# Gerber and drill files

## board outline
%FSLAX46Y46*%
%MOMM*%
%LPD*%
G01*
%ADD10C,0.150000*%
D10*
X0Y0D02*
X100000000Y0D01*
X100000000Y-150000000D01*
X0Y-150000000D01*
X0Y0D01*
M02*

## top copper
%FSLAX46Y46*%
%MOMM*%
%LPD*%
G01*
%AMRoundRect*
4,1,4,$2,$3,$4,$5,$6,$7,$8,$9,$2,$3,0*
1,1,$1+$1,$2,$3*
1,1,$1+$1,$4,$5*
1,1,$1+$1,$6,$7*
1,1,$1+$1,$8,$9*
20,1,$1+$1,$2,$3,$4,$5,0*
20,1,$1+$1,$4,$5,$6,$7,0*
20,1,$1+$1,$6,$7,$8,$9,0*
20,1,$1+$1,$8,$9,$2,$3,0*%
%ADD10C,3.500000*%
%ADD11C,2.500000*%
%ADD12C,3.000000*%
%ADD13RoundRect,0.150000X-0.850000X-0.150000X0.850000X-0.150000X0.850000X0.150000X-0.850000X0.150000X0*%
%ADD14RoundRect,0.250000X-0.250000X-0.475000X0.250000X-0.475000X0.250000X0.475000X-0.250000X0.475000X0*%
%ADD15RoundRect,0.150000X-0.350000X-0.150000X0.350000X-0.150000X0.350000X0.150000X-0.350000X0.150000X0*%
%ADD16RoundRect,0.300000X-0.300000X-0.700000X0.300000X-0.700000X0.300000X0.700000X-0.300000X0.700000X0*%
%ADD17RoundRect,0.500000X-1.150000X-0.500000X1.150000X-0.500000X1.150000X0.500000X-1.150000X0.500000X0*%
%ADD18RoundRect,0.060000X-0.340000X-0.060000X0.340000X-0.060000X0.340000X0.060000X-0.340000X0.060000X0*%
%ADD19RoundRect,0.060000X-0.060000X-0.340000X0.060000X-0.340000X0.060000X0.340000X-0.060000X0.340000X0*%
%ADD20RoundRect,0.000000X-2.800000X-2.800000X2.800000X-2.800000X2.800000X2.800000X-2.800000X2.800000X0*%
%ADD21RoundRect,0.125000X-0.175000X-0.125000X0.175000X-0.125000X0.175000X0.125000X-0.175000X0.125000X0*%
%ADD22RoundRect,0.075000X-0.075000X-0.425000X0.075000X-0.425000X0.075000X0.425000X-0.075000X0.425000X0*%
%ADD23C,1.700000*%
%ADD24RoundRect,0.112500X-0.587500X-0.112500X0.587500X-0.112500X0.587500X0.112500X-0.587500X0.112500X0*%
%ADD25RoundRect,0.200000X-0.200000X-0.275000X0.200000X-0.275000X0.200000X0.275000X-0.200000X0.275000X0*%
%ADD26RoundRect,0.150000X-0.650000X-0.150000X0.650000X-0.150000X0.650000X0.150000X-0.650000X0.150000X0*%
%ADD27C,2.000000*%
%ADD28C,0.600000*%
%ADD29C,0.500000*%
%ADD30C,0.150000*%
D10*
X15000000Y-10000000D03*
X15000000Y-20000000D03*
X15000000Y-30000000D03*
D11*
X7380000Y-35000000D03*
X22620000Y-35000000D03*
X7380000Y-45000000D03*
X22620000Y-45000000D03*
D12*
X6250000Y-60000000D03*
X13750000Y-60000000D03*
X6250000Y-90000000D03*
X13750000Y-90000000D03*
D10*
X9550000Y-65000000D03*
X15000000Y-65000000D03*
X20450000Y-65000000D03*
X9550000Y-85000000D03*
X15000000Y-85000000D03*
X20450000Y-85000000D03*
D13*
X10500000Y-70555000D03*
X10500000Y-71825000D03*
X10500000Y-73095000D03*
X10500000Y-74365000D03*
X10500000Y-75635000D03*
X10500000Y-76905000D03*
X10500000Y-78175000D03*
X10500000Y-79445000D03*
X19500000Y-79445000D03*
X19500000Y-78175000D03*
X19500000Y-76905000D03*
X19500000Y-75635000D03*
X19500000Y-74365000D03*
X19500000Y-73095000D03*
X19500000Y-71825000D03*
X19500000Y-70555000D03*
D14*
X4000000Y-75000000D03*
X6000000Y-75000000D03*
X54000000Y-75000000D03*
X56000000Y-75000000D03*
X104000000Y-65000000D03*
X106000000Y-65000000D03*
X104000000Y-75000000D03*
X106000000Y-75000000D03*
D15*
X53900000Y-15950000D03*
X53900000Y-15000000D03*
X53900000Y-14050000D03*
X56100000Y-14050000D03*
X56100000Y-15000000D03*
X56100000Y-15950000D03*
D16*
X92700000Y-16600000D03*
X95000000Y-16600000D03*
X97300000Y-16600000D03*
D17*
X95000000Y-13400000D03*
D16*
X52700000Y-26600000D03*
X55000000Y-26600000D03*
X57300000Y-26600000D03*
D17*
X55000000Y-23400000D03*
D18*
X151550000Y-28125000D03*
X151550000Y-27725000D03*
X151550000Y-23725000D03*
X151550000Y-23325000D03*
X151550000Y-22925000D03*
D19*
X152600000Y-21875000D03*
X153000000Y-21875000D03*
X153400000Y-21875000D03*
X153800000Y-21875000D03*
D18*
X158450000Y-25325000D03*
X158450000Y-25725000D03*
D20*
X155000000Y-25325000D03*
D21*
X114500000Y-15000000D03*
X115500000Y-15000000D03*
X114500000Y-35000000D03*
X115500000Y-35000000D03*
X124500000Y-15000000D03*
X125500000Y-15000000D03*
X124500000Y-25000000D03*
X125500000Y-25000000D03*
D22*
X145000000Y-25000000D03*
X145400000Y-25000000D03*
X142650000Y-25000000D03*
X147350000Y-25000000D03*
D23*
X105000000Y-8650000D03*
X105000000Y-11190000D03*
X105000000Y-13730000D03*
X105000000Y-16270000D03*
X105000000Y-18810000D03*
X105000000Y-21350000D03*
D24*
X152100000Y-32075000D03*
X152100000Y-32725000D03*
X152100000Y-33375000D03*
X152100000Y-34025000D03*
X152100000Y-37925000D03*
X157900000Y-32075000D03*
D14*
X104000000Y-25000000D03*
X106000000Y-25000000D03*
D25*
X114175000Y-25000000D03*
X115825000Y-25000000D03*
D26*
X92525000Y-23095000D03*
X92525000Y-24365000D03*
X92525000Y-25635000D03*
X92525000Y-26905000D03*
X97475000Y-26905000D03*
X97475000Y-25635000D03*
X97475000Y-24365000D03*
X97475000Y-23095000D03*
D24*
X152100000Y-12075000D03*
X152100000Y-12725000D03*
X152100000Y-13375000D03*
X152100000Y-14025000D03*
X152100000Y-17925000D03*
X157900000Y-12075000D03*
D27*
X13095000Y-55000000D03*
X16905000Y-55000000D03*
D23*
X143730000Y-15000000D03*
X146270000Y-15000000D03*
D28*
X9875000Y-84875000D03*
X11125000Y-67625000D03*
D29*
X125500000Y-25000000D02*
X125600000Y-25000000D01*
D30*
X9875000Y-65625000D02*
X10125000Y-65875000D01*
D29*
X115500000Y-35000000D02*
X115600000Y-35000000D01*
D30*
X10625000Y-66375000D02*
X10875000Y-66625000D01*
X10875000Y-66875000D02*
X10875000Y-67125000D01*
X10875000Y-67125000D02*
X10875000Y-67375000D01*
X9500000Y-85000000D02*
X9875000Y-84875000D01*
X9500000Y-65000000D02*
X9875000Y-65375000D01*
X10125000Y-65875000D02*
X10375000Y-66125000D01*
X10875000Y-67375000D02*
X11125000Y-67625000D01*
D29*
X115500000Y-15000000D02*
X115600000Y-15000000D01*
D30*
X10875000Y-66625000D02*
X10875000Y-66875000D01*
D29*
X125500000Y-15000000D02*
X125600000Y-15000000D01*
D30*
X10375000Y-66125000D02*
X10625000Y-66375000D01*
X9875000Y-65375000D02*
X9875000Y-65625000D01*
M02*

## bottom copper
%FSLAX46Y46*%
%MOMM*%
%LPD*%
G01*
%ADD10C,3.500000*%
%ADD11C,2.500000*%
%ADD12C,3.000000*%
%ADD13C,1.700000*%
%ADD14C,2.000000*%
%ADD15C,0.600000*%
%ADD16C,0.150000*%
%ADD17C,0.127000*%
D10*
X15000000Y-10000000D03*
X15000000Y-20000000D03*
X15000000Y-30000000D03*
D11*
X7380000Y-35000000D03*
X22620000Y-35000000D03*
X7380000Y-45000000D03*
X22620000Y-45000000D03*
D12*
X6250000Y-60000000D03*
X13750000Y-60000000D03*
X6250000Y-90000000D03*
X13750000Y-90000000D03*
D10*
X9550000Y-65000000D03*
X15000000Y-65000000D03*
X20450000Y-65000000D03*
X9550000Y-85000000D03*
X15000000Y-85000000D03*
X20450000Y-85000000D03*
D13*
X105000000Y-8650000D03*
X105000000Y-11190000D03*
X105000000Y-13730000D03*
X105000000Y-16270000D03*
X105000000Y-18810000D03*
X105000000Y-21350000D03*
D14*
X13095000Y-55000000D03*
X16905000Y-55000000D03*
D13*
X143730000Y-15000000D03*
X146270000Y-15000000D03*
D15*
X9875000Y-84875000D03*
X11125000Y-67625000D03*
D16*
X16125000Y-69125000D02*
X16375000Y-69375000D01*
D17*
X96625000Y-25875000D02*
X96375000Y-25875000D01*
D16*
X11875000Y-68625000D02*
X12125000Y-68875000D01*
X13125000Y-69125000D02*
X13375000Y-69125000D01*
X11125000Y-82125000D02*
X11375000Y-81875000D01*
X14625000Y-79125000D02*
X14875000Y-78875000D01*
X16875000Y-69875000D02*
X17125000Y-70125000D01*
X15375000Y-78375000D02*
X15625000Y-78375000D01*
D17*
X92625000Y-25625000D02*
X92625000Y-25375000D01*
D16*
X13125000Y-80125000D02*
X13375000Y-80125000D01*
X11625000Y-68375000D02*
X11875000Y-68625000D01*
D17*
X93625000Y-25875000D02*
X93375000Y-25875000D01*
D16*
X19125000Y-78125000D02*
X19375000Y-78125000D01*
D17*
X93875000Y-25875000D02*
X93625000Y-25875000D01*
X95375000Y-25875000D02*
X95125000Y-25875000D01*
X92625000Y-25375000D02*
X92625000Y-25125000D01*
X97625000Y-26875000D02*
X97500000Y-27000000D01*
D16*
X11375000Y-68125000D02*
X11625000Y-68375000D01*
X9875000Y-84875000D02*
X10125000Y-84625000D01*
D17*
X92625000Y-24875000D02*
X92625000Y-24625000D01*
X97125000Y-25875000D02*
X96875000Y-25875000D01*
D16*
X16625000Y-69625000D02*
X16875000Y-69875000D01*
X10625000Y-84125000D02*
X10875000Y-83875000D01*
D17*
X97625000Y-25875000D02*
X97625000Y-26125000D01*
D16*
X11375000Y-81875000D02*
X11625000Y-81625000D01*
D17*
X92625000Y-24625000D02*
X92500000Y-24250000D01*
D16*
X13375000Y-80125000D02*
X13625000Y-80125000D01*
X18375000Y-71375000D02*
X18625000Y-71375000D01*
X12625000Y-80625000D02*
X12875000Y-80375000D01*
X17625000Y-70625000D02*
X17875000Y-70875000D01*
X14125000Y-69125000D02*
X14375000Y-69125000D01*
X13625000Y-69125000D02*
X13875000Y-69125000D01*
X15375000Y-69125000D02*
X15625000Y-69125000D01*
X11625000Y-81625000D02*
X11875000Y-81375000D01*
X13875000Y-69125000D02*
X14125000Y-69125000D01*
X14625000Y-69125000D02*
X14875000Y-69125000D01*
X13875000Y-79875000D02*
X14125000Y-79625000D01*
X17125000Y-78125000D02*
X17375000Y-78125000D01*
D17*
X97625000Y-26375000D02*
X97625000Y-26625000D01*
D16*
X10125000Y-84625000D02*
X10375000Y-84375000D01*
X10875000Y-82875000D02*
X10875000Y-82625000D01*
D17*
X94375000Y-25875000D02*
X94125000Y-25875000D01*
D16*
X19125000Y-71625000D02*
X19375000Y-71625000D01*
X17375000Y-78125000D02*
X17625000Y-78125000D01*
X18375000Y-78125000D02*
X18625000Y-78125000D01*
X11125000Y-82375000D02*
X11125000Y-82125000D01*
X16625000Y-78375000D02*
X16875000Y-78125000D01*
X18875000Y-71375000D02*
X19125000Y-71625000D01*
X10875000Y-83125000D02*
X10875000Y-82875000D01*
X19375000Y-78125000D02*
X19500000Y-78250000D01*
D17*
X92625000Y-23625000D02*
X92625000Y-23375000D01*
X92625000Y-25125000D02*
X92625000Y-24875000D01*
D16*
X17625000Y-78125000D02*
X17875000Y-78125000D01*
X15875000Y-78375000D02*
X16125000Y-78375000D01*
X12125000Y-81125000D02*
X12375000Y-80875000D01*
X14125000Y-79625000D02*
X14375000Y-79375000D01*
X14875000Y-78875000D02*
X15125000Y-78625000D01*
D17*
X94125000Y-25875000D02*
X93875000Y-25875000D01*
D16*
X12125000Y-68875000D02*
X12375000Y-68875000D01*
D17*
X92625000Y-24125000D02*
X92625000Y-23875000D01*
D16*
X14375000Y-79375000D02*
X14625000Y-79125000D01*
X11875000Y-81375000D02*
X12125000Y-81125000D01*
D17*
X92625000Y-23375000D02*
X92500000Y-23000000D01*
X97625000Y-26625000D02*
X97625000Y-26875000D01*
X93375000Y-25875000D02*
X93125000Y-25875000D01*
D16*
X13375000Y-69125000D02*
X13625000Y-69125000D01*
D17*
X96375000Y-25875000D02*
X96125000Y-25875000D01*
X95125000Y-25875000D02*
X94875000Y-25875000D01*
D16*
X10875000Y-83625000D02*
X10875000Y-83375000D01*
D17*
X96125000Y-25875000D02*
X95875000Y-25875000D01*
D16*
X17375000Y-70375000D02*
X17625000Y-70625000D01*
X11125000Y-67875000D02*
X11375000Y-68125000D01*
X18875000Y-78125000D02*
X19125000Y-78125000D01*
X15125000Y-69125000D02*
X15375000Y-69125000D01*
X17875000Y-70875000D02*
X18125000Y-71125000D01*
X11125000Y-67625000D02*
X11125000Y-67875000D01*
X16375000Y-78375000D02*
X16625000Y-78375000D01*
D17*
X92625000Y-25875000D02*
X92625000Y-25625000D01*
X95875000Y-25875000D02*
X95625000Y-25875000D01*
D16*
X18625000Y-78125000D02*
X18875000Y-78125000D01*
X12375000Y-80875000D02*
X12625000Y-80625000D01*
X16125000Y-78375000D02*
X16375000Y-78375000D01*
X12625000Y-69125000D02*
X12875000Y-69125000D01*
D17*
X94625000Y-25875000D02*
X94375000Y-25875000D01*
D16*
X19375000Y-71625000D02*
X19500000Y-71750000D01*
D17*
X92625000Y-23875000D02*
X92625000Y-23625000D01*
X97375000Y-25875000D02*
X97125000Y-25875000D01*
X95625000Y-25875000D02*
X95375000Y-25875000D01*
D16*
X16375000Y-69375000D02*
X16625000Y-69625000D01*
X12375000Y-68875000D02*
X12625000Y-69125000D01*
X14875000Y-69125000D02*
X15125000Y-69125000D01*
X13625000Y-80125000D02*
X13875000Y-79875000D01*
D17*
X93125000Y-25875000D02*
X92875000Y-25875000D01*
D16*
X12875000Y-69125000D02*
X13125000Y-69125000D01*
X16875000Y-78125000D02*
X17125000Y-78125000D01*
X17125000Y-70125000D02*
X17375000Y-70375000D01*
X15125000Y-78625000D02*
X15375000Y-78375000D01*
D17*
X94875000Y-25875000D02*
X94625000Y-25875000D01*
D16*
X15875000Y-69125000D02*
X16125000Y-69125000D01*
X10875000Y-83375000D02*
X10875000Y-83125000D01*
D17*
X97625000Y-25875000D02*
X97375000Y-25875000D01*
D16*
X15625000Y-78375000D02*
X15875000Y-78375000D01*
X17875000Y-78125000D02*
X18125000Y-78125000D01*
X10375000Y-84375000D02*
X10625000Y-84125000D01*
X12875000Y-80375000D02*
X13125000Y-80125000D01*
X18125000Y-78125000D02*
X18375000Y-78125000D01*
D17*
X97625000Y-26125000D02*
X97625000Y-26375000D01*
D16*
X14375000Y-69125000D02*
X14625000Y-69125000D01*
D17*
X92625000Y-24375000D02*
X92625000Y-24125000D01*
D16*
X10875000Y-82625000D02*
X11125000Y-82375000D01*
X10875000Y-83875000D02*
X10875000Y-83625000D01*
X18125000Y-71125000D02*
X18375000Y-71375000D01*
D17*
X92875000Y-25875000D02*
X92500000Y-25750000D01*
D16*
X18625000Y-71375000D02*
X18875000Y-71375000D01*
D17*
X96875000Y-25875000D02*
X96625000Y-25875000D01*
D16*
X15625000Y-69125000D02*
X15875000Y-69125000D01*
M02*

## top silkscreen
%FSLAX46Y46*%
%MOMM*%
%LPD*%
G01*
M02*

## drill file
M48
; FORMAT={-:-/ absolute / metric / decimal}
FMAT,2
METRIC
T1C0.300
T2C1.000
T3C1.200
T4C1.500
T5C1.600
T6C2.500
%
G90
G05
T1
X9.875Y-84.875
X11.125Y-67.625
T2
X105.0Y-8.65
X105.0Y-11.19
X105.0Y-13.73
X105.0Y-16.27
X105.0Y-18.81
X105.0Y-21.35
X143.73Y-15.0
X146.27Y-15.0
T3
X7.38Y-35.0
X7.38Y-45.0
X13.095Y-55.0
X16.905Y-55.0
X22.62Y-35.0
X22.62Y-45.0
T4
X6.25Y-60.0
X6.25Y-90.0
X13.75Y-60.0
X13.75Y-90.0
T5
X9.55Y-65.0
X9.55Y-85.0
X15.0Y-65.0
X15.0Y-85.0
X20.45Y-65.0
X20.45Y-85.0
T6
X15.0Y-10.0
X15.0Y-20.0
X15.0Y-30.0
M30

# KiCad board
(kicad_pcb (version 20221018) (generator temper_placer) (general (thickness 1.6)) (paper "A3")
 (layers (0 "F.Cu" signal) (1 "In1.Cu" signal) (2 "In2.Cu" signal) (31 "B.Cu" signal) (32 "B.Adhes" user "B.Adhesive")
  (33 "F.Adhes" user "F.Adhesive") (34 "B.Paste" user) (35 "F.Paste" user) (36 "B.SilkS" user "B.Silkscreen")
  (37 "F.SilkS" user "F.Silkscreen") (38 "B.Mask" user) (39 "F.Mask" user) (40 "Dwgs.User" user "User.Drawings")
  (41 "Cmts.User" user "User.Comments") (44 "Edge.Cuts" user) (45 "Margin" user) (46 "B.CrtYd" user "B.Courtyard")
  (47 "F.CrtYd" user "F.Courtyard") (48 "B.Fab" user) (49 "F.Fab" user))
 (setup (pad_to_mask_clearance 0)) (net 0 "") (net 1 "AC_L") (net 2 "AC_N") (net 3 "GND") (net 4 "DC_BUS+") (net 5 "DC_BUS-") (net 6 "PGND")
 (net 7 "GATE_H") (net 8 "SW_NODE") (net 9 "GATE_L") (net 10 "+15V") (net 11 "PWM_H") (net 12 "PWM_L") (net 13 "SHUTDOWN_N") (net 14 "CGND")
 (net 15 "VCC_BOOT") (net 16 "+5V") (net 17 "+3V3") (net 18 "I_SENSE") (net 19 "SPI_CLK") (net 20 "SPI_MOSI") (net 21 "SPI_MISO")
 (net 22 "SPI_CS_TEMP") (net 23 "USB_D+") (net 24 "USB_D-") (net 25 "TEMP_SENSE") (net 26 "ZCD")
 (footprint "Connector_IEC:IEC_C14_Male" (layer "F.Cu") (at 15 10 0) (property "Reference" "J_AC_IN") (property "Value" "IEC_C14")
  (pad "1" thru_hole circle (at 0 0) (size 3.5 3.5) (drill 2.5) (layers *.Cu *.Mask) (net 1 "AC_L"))
  (pad "2" thru_hole circle (at 0 10) (size 3.5 3.5) (drill 2.5) (layers *.Cu *.Mask) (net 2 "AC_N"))
  (pad "3" thru_hole circle (at 0 20) (size 3.5 3.5) (drill 2.5) (layers *.Cu *.Mask) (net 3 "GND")))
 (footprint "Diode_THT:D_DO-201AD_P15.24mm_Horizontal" (layer "F.Cu") (at 7.38 35 0) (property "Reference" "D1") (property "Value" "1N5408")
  (pad "1" thru_hole circle (at 0 0) (size 2.5 2.5) (drill 1.2) (layers *.Cu *.Mask) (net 1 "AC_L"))
  (pad "2" thru_hole circle (at 15.24 0) (size 2.5 2.5) (drill 1.2) (layers *.Cu *.Mask) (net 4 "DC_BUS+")))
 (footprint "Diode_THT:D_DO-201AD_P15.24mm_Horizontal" (layer "F.Cu") (at 7.38 45 0) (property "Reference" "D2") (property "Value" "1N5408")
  (pad "1" thru_hole circle (at 0 0) (size 2.5 2.5) (drill 1.2) (layers *.Cu *.Mask) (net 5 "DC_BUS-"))
  (pad "2" thru_hole circle (at 15.24 0) (size 2.5 2.5) (drill 1.2) (layers *.Cu *.Mask) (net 2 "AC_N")))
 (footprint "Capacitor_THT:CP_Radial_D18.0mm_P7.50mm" (layer "F.Cu") (at 6.25 60 0) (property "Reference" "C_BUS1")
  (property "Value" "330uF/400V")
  (pad "1" thru_hole circle (at 0 0) (size 3 3) (drill 1.5) (layers *.Cu *.Mask) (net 4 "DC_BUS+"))
  (pad "2" thru_hole circle (at 7.5 0) (size 3 3) (drill 1.5) (layers *.Cu *.Mask) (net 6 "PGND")))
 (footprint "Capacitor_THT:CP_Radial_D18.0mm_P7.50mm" (layer "F.Cu") (at 6.25 90 0) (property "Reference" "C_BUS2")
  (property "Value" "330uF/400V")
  (pad "1" thru_hole circle (at 0 0) (size 3 3) (drill 1.5) (layers *.Cu *.Mask) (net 6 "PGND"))
  (pad "2" thru_hole circle (at 7.5 0) (size 3 3) (drill 1.5) (layers *.Cu *.Mask) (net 5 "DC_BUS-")))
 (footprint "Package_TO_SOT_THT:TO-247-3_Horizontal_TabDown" (layer "F.Cu") (at 9.55 65 0) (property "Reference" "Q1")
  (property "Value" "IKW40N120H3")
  (pad "1" thru_hole circle (at 0 0) (size 3.5 3.5) (drill 1.6) (layers *.Cu *.Mask) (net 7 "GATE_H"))
  (pad "2" thru_hole circle (at 5.45 0) (size 3.5 3.5) (drill 1.6) (layers *.Cu *.Mask) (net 4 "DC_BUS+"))
  (pad "3" thru_hole circle (at 10.9 0) (size 3.5 3.5) (drill 1.6) (layers *.Cu *.Mask) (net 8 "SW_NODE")))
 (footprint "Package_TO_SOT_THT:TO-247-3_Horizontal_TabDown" (layer "F.Cu") (at 9.55 85 0) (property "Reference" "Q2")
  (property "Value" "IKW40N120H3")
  (pad "1" thru_hole circle (at 0 0) (size 3.5 3.5) (drill 1.6) (layers *.Cu *.Mask) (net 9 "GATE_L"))
  (pad "2" thru_hole circle (at 5.45 0) (size 3.5 3.5) (drill 1.6) (layers *.Cu *.Mask) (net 8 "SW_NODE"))
  (pad "3" thru_hole circle (at 10.9 0) (size 3.5 3.5) (drill 1.6) (layers *.Cu *.Mask) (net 5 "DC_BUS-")))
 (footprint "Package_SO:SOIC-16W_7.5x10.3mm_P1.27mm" (layer "F.Cu") (at 15 75 0) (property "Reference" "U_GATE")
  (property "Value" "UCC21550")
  (pad "1" smd roundrect (at -4.5 -4.445) (size 2 0.6) (layers "F.Cu" "F.Paste" "F.Mask") (roundrect_rratio 0.25) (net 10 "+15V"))
  (pad "2" smd roundrect (at -4.5 -3.175) (size 2 0.6) (layers "F.Cu" "F.Paste" "F.Mask") (roundrect_rratio 0.25) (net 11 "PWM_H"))
  (pad "3" smd roundrect (at -4.5 -1.905) (size 2 0.6) (layers "F.Cu" "F.Paste" "F.Mask") (roundrect_rratio 0.25) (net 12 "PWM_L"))
  (pad "4" smd roundrect (at -4.5 -0.635) (size 2 0.6) (layers "F.Cu" "F.Paste" "F.Mask") (roundrect_rratio 0.25) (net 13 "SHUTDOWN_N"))
  (pad "5" smd roundrect (at -4.5 0.635) (size 2 0.6) (layers "F.Cu" "F.Paste" "F.Mask") (roundrect_rratio 0.25) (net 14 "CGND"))
  (pad "6" smd roundrect (at -4.5 1.905) (size 2 0.6) (layers "F.Cu" "F.Paste" "F.Mask") (roundrect_rratio 0.25) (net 14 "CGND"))
  (pad "7" smd roundrect (at -4.5 3.175) (size 2 0.6) (layers "F.Cu" "F.Paste" "F.Mask") (roundrect_rratio 0.25) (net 14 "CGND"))
  (pad "8" smd roundrect (at -4.5 4.445) (size 2 0.6) (layers "F.Cu" "F.Paste" "F.Mask") (roundrect_rratio 0.25) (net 14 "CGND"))
  (pad "9" smd roundrect (at 4.5 4.445) (size 2 0.6) (layers "F.Cu" "F.Paste" "F.Mask") (roundrect_rratio 0.25) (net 8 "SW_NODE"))
  (pad "10" smd roundrect (at 4.5 3.175) (size 2 0.6) (layers "F.Cu" "F.Paste" "F.Mask") (roundrect_rratio 0.25) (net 9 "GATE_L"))
  (pad "11" smd roundrect (at 4.5 1.905) (size 2 0.6) (layers "F.Cu" "F.Paste" "F.Mask") (roundrect_rratio 0.25) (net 10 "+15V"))
  (pad "12" smd roundrect (at 4.5 0.635) (size 2 0.6) (layers "F.Cu" "F.Paste" "F.Mask") (roundrect_rratio 0.25) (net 6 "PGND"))
  (pad "13" smd roundrect (at 4.5 -0.635) (size 2 0.6) (layers "F.Cu" "F.Paste" "F.Mask") (roundrect_rratio 0.25) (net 6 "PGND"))
  (pad "14" smd roundrect (at 4.5 -1.905) (size 2 0.6) (layers "F.Cu" "F.Paste" "F.Mask") (roundrect_rratio 0.25) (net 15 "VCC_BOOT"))
  (pad "15" smd roundrect (at 4.5 -3.175) (size 2 0.6) (layers "F.Cu" "F.Paste" "F.Mask") (roundrect_rratio 0.25) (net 7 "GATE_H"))
  (pad "16" smd roundrect (at 4.5 -4.445) (size 2 0.6) (layers "F.Cu" "F.Paste" "F.Mask") (roundrect_rratio 0.25) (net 8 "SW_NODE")))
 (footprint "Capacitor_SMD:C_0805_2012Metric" (layer "F.Cu") (at 5 75 0) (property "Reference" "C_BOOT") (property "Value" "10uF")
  (pad "1" smd roundrect (at -1 0) (size 1 1.45) (layers "F.Cu" "F.Paste" "F.Mask") (roundrect_rratio 0.25) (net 15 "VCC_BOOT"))
  (pad "2" smd roundrect (at 1 0) (size 1 1.45) (layers "F.Cu" "F.Paste" "F.Mask") (roundrect_rratio 0.25) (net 8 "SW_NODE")))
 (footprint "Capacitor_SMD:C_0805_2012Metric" (layer "F.Cu") (at 55 75 0) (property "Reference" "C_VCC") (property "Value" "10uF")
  (pad "1" smd roundrect (at -1 0) (size 1 1.45) (layers "F.Cu" "F.Paste" "F.Mask") (roundrect_rratio 0.25) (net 10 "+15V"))
  (pad "2" smd roundrect (at 1 0) (size 1 1.45) (layers "F.Cu" "F.Paste" "F.Mask") (roundrect_rratio 0.25) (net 14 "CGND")))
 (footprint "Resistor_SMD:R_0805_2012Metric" (layer "F.Cu") (at 105 65 0) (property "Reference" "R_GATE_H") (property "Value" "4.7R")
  (pad "1" smd roundrect (at -1 0) (size 1 1.45) (layers "F.Cu" "F.Paste" "F.Mask") (roundrect_rratio 0.25) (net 7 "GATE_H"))
  (pad "2" smd roundrect (at 1 0) (size 1 1.45) (layers "F.Cu" "F.Paste" "F.Mask") (roundrect_rratio 0.25) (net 7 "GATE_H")))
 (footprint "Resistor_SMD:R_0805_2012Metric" (layer "F.Cu") (at 105 75 0) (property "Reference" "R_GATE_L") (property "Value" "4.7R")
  (pad "1" smd roundrect (at -1 0) (size 1 1.45) (layers "F.Cu" "F.Paste" "F.Mask") (roundrect_rratio 0.25) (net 9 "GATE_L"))
  (pad "2" smd roundrect (at 1 0) (size 1 1.45) (layers "F.Cu" "F.Paste" "F.Mask") (roundrect_rratio 0.25) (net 9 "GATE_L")))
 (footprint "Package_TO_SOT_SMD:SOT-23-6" (layer "F.Cu") (at 55 15 0) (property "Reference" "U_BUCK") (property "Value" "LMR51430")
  (pad "1" smd roundrect (at -1.1 0.95) (size 1 0.6) (layers "F.Cu" "F.Paste" "F.Mask") (roundrect_rratio 0.25) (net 3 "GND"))
  (pad "2" smd roundrect (at -1.1 0) (size 1 0.6) (layers "F.Cu" "F.Paste" "F.Mask") (roundrect_rratio 0.25) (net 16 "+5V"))
  (pad "3" smd roundrect (at -1.1 -0.95) (size 1 0.6) (layers "F.Cu" "F.Paste" "F.Mask") (roundrect_rratio 0.25) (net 10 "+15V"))
  (pad "4" smd roundrect (at 1.1 -0.95) (size 1 0.6) (layers "F.Cu" "F.Paste" "F.Mask") (roundrect_rratio 0.25) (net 16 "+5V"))
  (pad "5" smd roundrect (at 1.1 0) (size 1 0.6) (layers "F.Cu" "F.Paste" "F.Mask") (roundrect_rratio 0.25) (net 3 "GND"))
  (pad "6" smd roundrect (at 1.1 0.95) (size 1 0.6) (layers "F.Cu" "F.Paste" "F.Mask") (roundrect_rratio 0.25) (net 3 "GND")))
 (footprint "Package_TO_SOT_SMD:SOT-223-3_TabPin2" (layer "F.Cu") (at 95 16.6 0) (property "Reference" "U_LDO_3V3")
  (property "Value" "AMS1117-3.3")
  (pad "1" smd roundrect (at -2.3 0) (size 1.2 2) (layers "F.Cu" "F.Paste" "F.Mask") (roundrect_rratio 0.25) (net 3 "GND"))
  (pad "2" smd roundrect (at 0 0) (size 1.2 2) (layers "F.Cu" "F.Paste" "F.Mask") (roundrect_rratio 0.25) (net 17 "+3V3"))
  (pad "3" smd roundrect (at 2.3 0) (size 1.2 2) (layers "F.Cu" "F.Paste" "F.Mask") (roundrect_rratio 0.25) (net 16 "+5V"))
  (pad "4" smd roundrect (at 0 -3.2) (size 3.3 2) (layers "F.Cu" "F.Paste" "F.Mask") (roundrect_rratio 0.25) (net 17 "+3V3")))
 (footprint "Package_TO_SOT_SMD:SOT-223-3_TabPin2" (layer "F.Cu") (at 55 26.6 0) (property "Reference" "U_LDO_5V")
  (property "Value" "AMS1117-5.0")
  (pad "1" smd roundrect (at -2.3 0) (size 1.2 2) (layers "F.Cu" "F.Paste" "F.Mask") (roundrect_rratio 0.25) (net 3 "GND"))
  (pad "2" smd roundrect (at 0 0) (size 1.2 2) (layers "F.Cu" "F.Paste" "F.Mask") (roundrect_rratio 0.25) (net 16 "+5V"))
  (pad "3" smd roundrect (at 2.3 0) (size 1.2 2) (layers "F.Cu" "F.Paste" "F.Mask") (roundrect_rratio 0.25) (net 10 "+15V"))
  (pad "4" smd roundrect (at 0 -3.2) (size 3.3 2) (layers "F.Cu" "F.Paste" "F.Mask") (roundrect_rratio 0.25) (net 16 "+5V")))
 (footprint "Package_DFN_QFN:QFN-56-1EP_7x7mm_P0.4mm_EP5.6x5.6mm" (layer "F.Cu") (at 155 25.325 0) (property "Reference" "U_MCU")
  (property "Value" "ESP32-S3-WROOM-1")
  (pad "1" smd roundrect (at -3.45 2.8) (size 0.8 0.24) (layers "F.Cu" "F.Paste" "F.Mask") (roundrect_rratio 0.25) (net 17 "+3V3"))
  (pad "2" smd roundrect (at -3.45 2.4) (size 0.8 0.24) (layers "F.Cu" "F.Paste" "F.Mask") (roundrect_rratio 0.25) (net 3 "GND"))
  (pad "13" smd roundrect (at -3.45 -1.6) (size 0.8 0.24) (layers "F.Cu" "F.Paste" "F.Mask") (roundrect_rratio 0.25) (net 11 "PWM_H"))
  (pad "14" smd roundrect (at -3.45 -2) (size 0.8 0.24) (layers "F.Cu" "F.Paste" "F.Mask") (roundrect_rratio 0.25) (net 12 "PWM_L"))
  (pad "15" smd roundrect (at -3.45 -2.4) (size 0.8 0.24) (layers "F.Cu" "F.Paste" "F.Mask") (roundrect_rratio 0.25) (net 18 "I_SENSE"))
  (pad "20" smd roundrect (at -2.4 -3.45) (size 0.24 0.8) (layers "F.Cu" "F.Paste" "F.Mask") (roundrect_rratio 0.25) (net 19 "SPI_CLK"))
  (pad "21" smd roundrect (at -2 -3.45) (size 0.24 0.8) (layers "F.Cu" "F.Paste" "F.Mask") (roundrect_rratio 0.25) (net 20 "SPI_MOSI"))
  (pad "22" smd roundrect (at -1.6 -3.45) (size 0.24 0.8) (layers "F.Cu" "F.Paste" "F.Mask") (roundrect_rratio 0.25) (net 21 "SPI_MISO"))
  (pad "23" smd roundrect (at -1.2 -3.45) (size 0.24 0.8) (layers "F.Cu" "F.Paste" "F.Mask") (roundrect_rratio 0.25) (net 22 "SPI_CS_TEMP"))
  (pad "40" smd roundrect (at 3.45 0) (size 0.8 0.24) (layers "F.Cu" "F.Paste" "F.Mask") (roundrect_rratio 0.25) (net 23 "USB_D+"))
  (pad "41" smd roundrect (at 3.45 0.4) (size 0.8 0.24) (layers "F.Cu" "F.Paste" "F.Mask") (roundrect_rratio 0.25) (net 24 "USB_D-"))
  (pad "57" smd roundrect (at 0 0) (size 5.6 5.6) (layers "F.Cu" "F.Paste" "F.Mask") (roundrect_rratio 0) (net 3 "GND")))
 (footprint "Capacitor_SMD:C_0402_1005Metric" (layer "F.Cu") (at 115 15 0) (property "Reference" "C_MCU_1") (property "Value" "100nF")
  (pad "1" smd roundrect (at -0.5 0) (size 0.6 0.5) (layers "F.Cu" "F.Paste" "F.Mask") (roundrect_rratio 0.25) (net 17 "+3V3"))
  (pad "2" smd roundrect (at 0.5 0) (size 0.6 0.5) (layers "F.Cu" "F.Paste" "F.Mask") (roundrect_rratio 0.25) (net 3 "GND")))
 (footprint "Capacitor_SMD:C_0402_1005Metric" (layer "F.Cu") (at 115 35 0) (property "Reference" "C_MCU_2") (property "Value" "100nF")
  (pad "1" smd roundrect (at -0.5 0) (size 0.6 0.5) (layers "F.Cu" "F.Paste" "F.Mask") (roundrect_rratio 0.25) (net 17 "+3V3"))
  (pad "2" smd roundrect (at 0.5 0) (size 0.6 0.5) (layers "F.Cu" "F.Paste" "F.Mask") (roundrect_rratio 0.25) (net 3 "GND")))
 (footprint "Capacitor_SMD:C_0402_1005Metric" (layer "F.Cu") (at 125 15 0) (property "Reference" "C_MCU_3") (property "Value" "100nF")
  (pad "1" smd roundrect (at -0.5 0) (size 0.6 0.5) (layers "F.Cu" "F.Paste" "F.Mask") (roundrect_rratio 0.25) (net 17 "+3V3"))
  (pad "2" smd roundrect (at 0.5 0) (size 0.6 0.5) (layers "F.Cu" "F.Paste" "F.Mask") (roundrect_rratio 0.25) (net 3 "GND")))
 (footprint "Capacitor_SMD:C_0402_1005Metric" (layer "F.Cu") (at 125 25 0) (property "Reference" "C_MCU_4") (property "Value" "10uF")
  (pad "1" smd roundrect (at -0.5 0) (size 0.6 0.5) (layers "F.Cu" "F.Paste" "F.Mask") (roundrect_rratio 0.25) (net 17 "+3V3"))
  (pad "2" smd roundrect (at 0.5 0) (size 0.6 0.5) (layers "F.Cu" "F.Paste" "F.Mask") (roundrect_rratio 0.25) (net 3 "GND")))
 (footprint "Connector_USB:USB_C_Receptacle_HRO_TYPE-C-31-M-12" (layer "F.Cu") (at 145 25 0) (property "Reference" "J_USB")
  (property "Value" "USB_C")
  (pad "A6" smd roundrect (at 0 0) (size 0.3 1) (layers "F.Cu" "F.Paste" "F.Mask") (roundrect_rratio 0.25) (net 23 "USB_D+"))
  (pad "B6" smd roundrect (at 0.4 0) (size 0.3 1) (layers "F.Cu" "F.Paste" "F.Mask") (roundrect_rratio 0.25) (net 24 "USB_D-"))
  (pad "A1" smd roundrect (at -2.35 0) (size 0.3 1) (layers "F.Cu" "F.Paste" "F.Mask") (roundrect_rratio 0.25) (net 3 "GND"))
  (pad "A12" smd roundrect (at 2.35 0) (size 0.3 1) (layers "F.Cu" "F.Paste" "F.Mask") (roundrect_rratio 0.25) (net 3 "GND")))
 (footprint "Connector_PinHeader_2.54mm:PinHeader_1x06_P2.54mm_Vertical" (layer "F.Cu") (at 105 8.65 0) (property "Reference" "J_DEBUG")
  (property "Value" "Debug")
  (pad "1" thru_hole circle (at 0 0) (size 1.7 1.7) (drill 1) (layers *.Cu *.Mask) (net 3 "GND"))
  (pad "2" thru_hole circle (at 0 2.54) (size 1.7 1.7) (drill 1) (layers *.Cu *.Mask) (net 17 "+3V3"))
  (pad "3" thru_hole circle (at 0 5.08) (size 1.7 1.7) (drill 1) (layers *.Cu *.Mask) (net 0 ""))
  (pad "4" thru_hole circle (at 0 7.62) (size 1.7 1.7) (drill 1) (layers *.Cu *.Mask) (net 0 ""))
  (pad "5" thru_hole circle (at 0 10.16) (size 1.7 1.7) (drill 1) (layers *.Cu *.Mask) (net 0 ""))
  (pad "6" thru_hole circle (at 0 12.7) (size 1.7 1.7) (drill 1) (layers *.Cu *.Mask) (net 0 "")))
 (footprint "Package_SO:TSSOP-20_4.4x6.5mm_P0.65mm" (layer "F.Cu") (at 155 35 0) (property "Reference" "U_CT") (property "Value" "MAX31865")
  (pad "1" smd roundrect (at -2.9 -2.925) (size 1.4 0.45) (layers "F.Cu" "F.Paste" "F.Mask") (roundrect_rratio 0.25) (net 19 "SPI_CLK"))
  (pad "2" smd roundrect (at -2.9 -2.275) (size 1.4 0.45) (layers "F.Cu" "F.Paste" "F.Mask") (roundrect_rratio 0.25) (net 20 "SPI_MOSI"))
  (pad "3" smd roundrect (at -2.9 -1.625) (size 1.4 0.45) (layers "F.Cu" "F.Paste" "F.Mask") (roundrect_rratio 0.25) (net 21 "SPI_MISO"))
  (pad "4" smd roundrect (at -2.9 -0.975) (size 1.4 0.45) (layers "F.Cu" "F.Paste" "F.Mask") (roundrect_rratio 0.25) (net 22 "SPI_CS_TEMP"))
  (pad "10" smd roundrect (at -2.9 2.925) (size 1.4 0.45) (layers "F.Cu" "F.Paste" "F.Mask") (roundrect_rratio 0.25) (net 3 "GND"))
  (pad "20" smd roundrect (at 2.9 -2.925) (size 1.4 0.45) (layers "F.Cu" "F.Paste" "F.Mask") (roundrect_rratio 0.25) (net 17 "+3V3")))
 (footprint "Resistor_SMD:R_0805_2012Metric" (layer "F.Cu") (at 105 25 0) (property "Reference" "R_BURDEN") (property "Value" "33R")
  (pad "1" smd roundrect (at -1 0) (size 1 1.45) (layers "F.Cu" "F.Paste" "F.Mask") (roundrect_rratio 0.25) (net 18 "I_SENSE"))
  (pad "2" smd roundrect (at 1 0) (size 1 1.45) (layers "F.Cu" "F.Paste" "F.Mask") (roundrect_rratio 0.25) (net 3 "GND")))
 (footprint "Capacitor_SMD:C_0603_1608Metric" (layer "F.Cu") (at 115 25 0) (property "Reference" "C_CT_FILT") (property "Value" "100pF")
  (pad "1" smd roundrect (at -0.825 0) (size 0.8 0.95) (layers "F.Cu" "F.Paste" "F.Mask") (roundrect_rratio 0.25) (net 18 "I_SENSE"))
  (pad "2" smd roundrect (at 0.825 0) (size 0.8 0.95) (layers "F.Cu" "F.Paste" "F.Mask") (roundrect_rratio 0.25) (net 3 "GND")))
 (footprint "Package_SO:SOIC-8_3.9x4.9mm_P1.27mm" (layer "F.Cu") (at 95 25 0) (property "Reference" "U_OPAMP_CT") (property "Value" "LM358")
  (pad "1" smd roundrect (at -2.475 -1.905) (size 1.6 0.6) (layers "F.Cu" "F.Paste" "F.Mask") (roundrect_rratio 0.25) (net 18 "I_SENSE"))
  (pad "2" smd roundrect (at -2.475 -0.635) (size 1.6 0.6) (layers "F.Cu" "F.Paste" "F.Mask") (roundrect_rratio 0.25) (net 18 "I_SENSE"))
  (pad "3" smd roundrect (at -2.475 0.635) (size 1.6 0.6) (layers "F.Cu" "F.Paste" "F.Mask") (roundrect_rratio 0.25) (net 18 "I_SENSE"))
  (pad "4" smd roundrect (at -2.475 1.905) (size 1.6 0.6) (layers "F.Cu" "F.Paste" "F.Mask") (roundrect_rratio 0.25) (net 3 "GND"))
  (pad "5" smd roundrect (at 2.475 1.905) (size 1.6 0.6) (layers "F.Cu" "F.Paste" "F.Mask") (roundrect_rratio 0.25) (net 18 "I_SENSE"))
  (pad "6" smd roundrect (at 2.475 0.635) (size 1.6 0.6) (layers "F.Cu" "F.Paste" "F.Mask") (roundrect_rratio 0.25) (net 18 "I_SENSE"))
  (pad "7" smd roundrect (at 2.475 -0.635) (size 1.6 0.6) (layers "F.Cu" "F.Paste" "F.Mask") (roundrect_rratio 0.25) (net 16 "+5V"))
  (pad "8" smd roundrect (at 2.475 -1.905) (size 1.6 0.6) (layers "F.Cu" "F.Paste" "F.Mask") (roundrect_rratio 0.25) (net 16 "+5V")))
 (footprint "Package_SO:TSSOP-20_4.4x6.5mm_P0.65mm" (layer "F.Cu") (at 155 15 0) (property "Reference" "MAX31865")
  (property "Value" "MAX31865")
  (pad "1" smd roundrect (at -2.9 -2.925) (size 1.4 0.45) (layers "F.Cu" "F.Paste" "F.Mask") (roundrect_rratio 0.25) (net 19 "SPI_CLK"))
  (pad "2" smd roundrect (at -2.9 -2.275) (size 1.4 0.45) (layers "F.Cu" "F.Paste" "F.Mask") (roundrect_rratio 0.25) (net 20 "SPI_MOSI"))
  (pad "3" smd roundrect (at -2.9 -1.625) (size 1.4 0.45) (layers "F.Cu" "F.Paste" "F.Mask") (roundrect_rratio 0.25) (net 21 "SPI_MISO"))
  (pad "4" smd roundrect (at -2.9 -0.975) (size 1.4 0.45) (layers "F.Cu" "F.Paste" "F.Mask") (roundrect_rratio 0.25) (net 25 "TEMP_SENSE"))
  (pad "10" smd roundrect (at -2.9 2.925) (size 1.4 0.45) (layers "F.Cu" "F.Paste" "F.Mask") (roundrect_rratio 0.25) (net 3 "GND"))
  (pad "20" smd roundrect (at 2.9 -2.925) (size 1.4 0.45) (layers "F.Cu" "F.Paste" "F.Mask") (roundrect_rratio 0.25) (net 17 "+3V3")))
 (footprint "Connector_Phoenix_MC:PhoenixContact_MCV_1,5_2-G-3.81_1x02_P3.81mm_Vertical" (layer "F.Cu") (at 13.095 55 0)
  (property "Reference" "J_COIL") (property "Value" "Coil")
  (pad "1" thru_hole circle (at 0 0) (size 2 2) (drill 1.2) (layers *.Cu *.Mask) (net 8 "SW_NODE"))
  (pad "2" thru_hole circle (at 3.81 0) (size 2 2) (drill 1.2) (layers *.Cu *.Mask) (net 3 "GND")))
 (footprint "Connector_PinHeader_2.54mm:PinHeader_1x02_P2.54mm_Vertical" (layer "F.Cu") (at 143.73 15 0) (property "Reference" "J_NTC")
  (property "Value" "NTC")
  (pad "1" thru_hole circle (at 0 0) (size 1.7 1.7) (drill 1) (layers *.Cu *.Mask) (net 25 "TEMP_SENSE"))
  (pad "2" thru_hole circle (at 2.54 0) (size 1.7 1.7) (drill 1) (layers *.Cu *.Mask) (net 3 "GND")))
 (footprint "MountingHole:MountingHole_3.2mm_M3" (layer "F.Cu") (at 105 5 0) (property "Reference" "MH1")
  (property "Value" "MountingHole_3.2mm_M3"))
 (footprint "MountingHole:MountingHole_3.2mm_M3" (layer "F.Cu") (at 105 35 0) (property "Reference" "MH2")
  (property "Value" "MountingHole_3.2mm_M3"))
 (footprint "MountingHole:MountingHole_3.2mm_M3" (layer "F.Cu") (at 105 45 0) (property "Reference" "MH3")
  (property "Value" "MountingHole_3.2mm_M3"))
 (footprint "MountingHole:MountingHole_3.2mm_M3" (layer "F.Cu") (at 105 55 0) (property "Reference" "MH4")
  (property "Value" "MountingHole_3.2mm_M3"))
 (gr_rect (start 0 0) (end 100 150) (layer "Edge.Cuts") (width 0.15))
 (segment (start 16.125 69.125) (end 16.375 69.375) (width 0.15) (layer "B.Cu") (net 7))
 (segment (start 96.625 25.875) (end 96.375 25.875) (width 0.127) (layer "B.Cu") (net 18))
 (segment (start 11.875 68.625) (end 12.125 68.875) (width 0.15) (layer "B.Cu") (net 7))
 (segment (start 13.125 69.125) (end 13.375 69.125) (width 0.15) (layer "B.Cu") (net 7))
 (segment (start 11.125 82.125) (end 11.375 81.875) (width 0.15) (layer "B.Cu") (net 9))
 (segment (start 14.625 79.125) (end 14.875 78.875) (width 0.15) (layer "B.Cu") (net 9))
 (segment (start 16.875 69.875) (end 17.125 70.125) (width 0.15) (layer "B.Cu") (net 7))
 (segment (start 125.5 25.0) (end 125.6 25.0) (width 0.5) (layer "F.Cu") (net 3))
 (segment (start 15.375 78.375) (end 15.625 78.375) (width 0.15) (layer "B.Cu") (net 9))
 (segment (start 92.625 25.625) (end 92.625 25.375) (width 0.127) (layer "B.Cu") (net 18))
 (segment (start 13.125 80.125) (end 13.375 80.125) (width 0.15) (layer "B.Cu") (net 9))
 (segment (start 11.625 68.375) (end 11.875 68.625) (width 0.15) (layer "B.Cu") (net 7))
 (segment (start 93.625 25.875) (end 93.375 25.875) (width 0.127) (layer "B.Cu") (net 18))
 (segment (start 19.125 78.125) (end 19.375 78.125) (width 0.15) (layer "B.Cu") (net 9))
 (segment (start 93.875 25.875) (end 93.625 25.875) (width 0.127) (layer "B.Cu") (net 18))
 (segment (start 95.375 25.875) (end 95.125 25.875) (width 0.127) (layer "B.Cu") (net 18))
 (segment (start 92.625 25.375) (end 92.625 25.125) (width 0.127) (layer "B.Cu") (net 18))
 (segment (start 97.625 26.875) (end 97.5 27.0) (width 0.127) (layer "B.Cu") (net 18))
 (segment (start 11.375 68.125) (end 11.625 68.375) (width 0.15) (layer "B.Cu") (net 7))
 (segment (start 9.875 84.875) (end 10.125 84.625) (width 0.15) (layer "B.Cu") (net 9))
 (segment (start 92.625 24.875) (end 92.625 24.625) (width 0.127) (layer "B.Cu") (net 18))
 (segment (start 97.125 25.875) (end 96.875 25.875) (width 0.127) (layer "B.Cu") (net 18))
 (segment (start 16.625 69.625) (end 16.875 69.875) (width 0.15) (layer "B.Cu") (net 7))
 (segment (start 10.625 84.125) (end 10.875 83.875) (width 0.15) (layer "B.Cu") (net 9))
 (segment (start 9.875 65.625) (end 10.125 65.875) (width 0.15) (layer "F.Cu") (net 7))
 (segment (start 97.625 25.875) (end 97.625 26.125) (width 0.127) (layer "B.Cu") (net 18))
 (segment (start 11.375 81.875) (end 11.625 81.625) (width 0.15) (layer "B.Cu") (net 9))
 (segment (start 92.625 24.625) (end 92.5 24.25) (width 0.127) (layer "B.Cu") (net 18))
 (segment (start 115.5 35.0) (end 115.6 35.0) (width 0.5) (layer "F.Cu") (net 3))
 (segment (start 13.375 80.125) (end 13.625 80.125) (width 0.15) (layer "B.Cu") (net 9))
 (segment (start 18.375 71.375) (end 18.625 71.375) (width 0.15) (layer "B.Cu") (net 7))
 (segment (start 12.625 80.625) (end 12.875 80.375) (width 0.15) (layer "B.Cu") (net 9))
 (segment (start 17.625 70.625) (end 17.875 70.875) (width 0.15) (layer "B.Cu") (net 7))
 (segment (start 14.125 69.125) (end 14.375 69.125) (width 0.15) (layer "B.Cu") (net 7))
 (segment (start 13.625 69.125) (end 13.875 69.125) (width 0.15) (layer "B.Cu") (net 7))
 (segment (start 15.375 69.125) (end 15.625 69.125) (width 0.15) (layer "B.Cu") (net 7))
 (segment (start 11.625 81.625) (end 11.875 81.375) (width 0.15) (layer "B.Cu") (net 9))
 (segment (start 10.625 66.375) (end 10.875 66.625) (width 0.15) (layer "F.Cu") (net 7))
 (segment (start 13.875 69.125) (end 14.125 69.125) (width 0.15) (layer "B.Cu") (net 7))
 (segment (start 14.625 69.125) (end 14.875 69.125) (width 0.15) (layer "B.Cu") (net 7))
 (segment (start 10.875 66.875) (end 10.875 67.125) (width 0.15) (layer "F.Cu") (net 7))
 (segment (start 13.875 79.875) (end 14.125 79.625) (width 0.15) (layer "B.Cu") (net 9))
 (segment (start 17.125 78.125) (end 17.375 78.125) (width 0.15) (layer "B.Cu") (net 9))
 (segment (start 97.625 26.375) (end 97.625 26.625) (width 0.127) (layer "B.Cu") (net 18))
 (segment (start 10.125 84.625) (end 10.375 84.375) (width 0.15) (layer "B.Cu") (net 9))
 (segment (start 10.875 82.875) (end 10.875 82.625) (width 0.15) (layer "B.Cu") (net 9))
 (segment (start 94.375 25.875) (end 94.125 25.875) (width 0.127) (layer "B.Cu") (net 18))
 (segment (start 19.125 71.625) (end 19.375 71.625) (width 0.15) (layer "B.Cu") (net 7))
 (segment (start 10.875 67.125) (end 10.875 67.375) (width 0.15) (layer "F.Cu") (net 7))
 (segment (start 17.375 78.125) (end 17.625 78.125) (width 0.15) (layer "B.Cu") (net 9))
 (segment (start 18.375 78.125) (end 18.625 78.125) (width 0.15) (layer "B.Cu") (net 9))
 (segment (start 11.125 82.375) (end 11.125 82.125) (width 0.15) (layer "B.Cu") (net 9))
 (segment (start 16.625 78.375) (end 16.875 78.125) (width 0.15) (layer "B.Cu") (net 9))
 (segment (start 18.875 71.375) (end 19.125 71.625) (width 0.15) (layer "B.Cu") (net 7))
 (segment (start 10.875 83.125) (end 10.875 82.875) (width 0.15) (layer "B.Cu") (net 9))
 (segment (start 19.375 78.125) (end 19.5 78.25) (width 0.15) (layer "B.Cu") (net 9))
 (segment (start 92.625 23.625) (end 92.625 23.375) (width 0.127) (layer "B.Cu") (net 18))
 (segment (start 92.625 25.125) (end 92.625 24.875) (width 0.127) (layer "B.Cu") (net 18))
 (segment (start 17.625 78.125) (end 17.875 78.125) (width 0.15) (layer "B.Cu") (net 9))
 (segment (start 9.5 85.0) (end 9.875 84.875) (width 0.15) (layer "F.Cu") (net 9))
 (segment (start 15.875 78.375) (end 16.125 78.375) (width 0.15) (layer "B.Cu") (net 9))
 (segment (start 9.5 65.0) (end 9.875 65.375) (width 0.15) (layer "F.Cu") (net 7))
 (segment (start 12.125 81.125) (end 12.375 80.875) (width 0.15) (layer "B.Cu") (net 9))
 (segment (start 14.125 79.625) (end 14.375 79.375) (width 0.15) (layer "B.Cu") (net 9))
 (segment (start 14.875 78.875) (end 15.125 78.625) (width 0.15) (layer "B.Cu") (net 9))
 (segment (start 94.125 25.875) (end 93.875 25.875) (width 0.127) (layer "B.Cu") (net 18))
 (segment (start 12.125 68.875) (end 12.375 68.875) (width 0.15) (layer "B.Cu") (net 7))
 (segment (start 92.625 24.125) (end 92.625 23.875) (width 0.127) (layer "B.Cu") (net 18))
 (segment (start 14.375 79.375) (end 14.625 79.125) (width 0.15) (layer "B.Cu") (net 9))
 (segment (start 11.875 81.375) (end 12.125 81.125) (width 0.15) (layer "B.Cu") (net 9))
 (segment (start 92.625 23.375) (end 92.5 23.0) (width 0.127) (layer "B.Cu") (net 18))
 (segment (start 10.125 65.875) (end 10.375 66.125) (width 0.15) (layer "F.Cu") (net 7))
 (segment (start 97.625 26.625) (end 97.625 26.875) (width 0.127) (layer "B.Cu") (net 18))
 (segment (start 93.375 25.875) (end 93.125 25.875) (width 0.127) (layer "B.Cu") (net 18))
 (segment (start 13.375 69.125) (end 13.625 69.125) (width 0.15) (layer "B.Cu") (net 7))
 (segment (start 96.375 25.875) (end 96.125 25.875) (width 0.127) (layer "B.Cu") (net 18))
 (segment (start 95.125 25.875) (end 94.875 25.875) (width 0.127) (layer "B.Cu") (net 18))
 (segment (start 10.875 83.625) (end 10.875 83.375) (width 0.15) (layer "B.Cu") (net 9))
 (segment (start 96.125 25.875) (end 95.875 25.875) (width 0.127) (layer "B.Cu") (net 18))
 (segment (start 17.375 70.375) (end 17.625 70.625) (width 0.15) (layer "B.Cu") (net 7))
 (segment (start 11.125 67.875) (end 11.375 68.125) (width 0.15) (layer "B.Cu") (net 7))
 (segment (start 18.875 78.125) (end 19.125 78.125) (width 0.15) (layer "B.Cu") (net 9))
 (segment (start 15.125 69.125) (end 15.375 69.125) (width 0.15) (layer "B.Cu") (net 7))
 (segment (start 17.875 70.875) (end 18.125 71.125) (width 0.15) (layer "B.Cu") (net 7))
 (segment (start 10.875 67.375) (end 11.125 67.625) (width 0.15) (layer "F.Cu") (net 7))
 (segment (start 11.125 67.625) (end 11.125 67.875) (width 0.15) (layer "B.Cu") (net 7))
 (segment (start 115.5 15.0) (end 115.6 15.0) (width 0.5) (layer "F.Cu") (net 3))
 (segment (start 16.375 78.375) (end 16.625 78.375) (width 0.15) (layer "B.Cu") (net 9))
 (segment (start 92.625 25.875) (end 92.625 25.625) (width 0.127) (layer "B.Cu") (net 18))
 (segment (start 10.875 66.625) (end 10.875 66.875) (width 0.15) (layer "F.Cu") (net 7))
 (segment (start 95.875 25.875) (end 95.625 25.875) (width 0.127) (layer "B.Cu") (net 18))
 (segment (start 18.625 78.125) (end 18.875 78.125) (width 0.15) (layer "B.Cu") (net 9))
 (segment (start 12.375 80.875) (end 12.625 80.625) (width 0.15) (layer "B.Cu") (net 9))
 (segment (start 125.5 15.0) (end 125.6 15.0) (width 0.5) (layer "F.Cu") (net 3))
 (segment (start 16.125 78.375) (end 16.375 78.375) (width 0.15) (layer "B.Cu") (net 9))
 (segment (start 12.625 69.125) (end 12.875 69.125) (width 0.15) (layer "B.Cu") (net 7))
 (segment (start 94.625 25.875) (end 94.375 25.875) (width 0.127) (layer "B.Cu") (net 18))
 (segment (start 19.375 71.625) (end 19.5 71.75) (width 0.15) (layer "B.Cu") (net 7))
 (segment (start 92.625 23.875) (end 92.625 23.625) (width 0.127) (layer "B.Cu") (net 18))
 (segment (start 97.375 25.875) (end 97.125 25.875) (width 0.127) (layer "B.Cu") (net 18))
 (segment (start 95.625 25.875) (end 95.375 25.875) (width 0.127) (layer "B.Cu") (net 18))
 (segment (start 16.375 69.375) (end 16.625 69.625) (width 0.15) (layer "B.Cu") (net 7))
 (segment (start 12.375 68.875) (end 12.625 69.125) (width 0.15) (layer "B.Cu") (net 7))
 (segment (start 10.375 66.125) (end 10.625 66.375) (width 0.15) (layer "F.Cu") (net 7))
 (segment (start 14.875 69.125) (end 15.125 69.125) (width 0.15) (layer "B.Cu") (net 7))
 (segment (start 13.625 80.125) (end 13.875 79.875) (width 0.15) (layer "B.Cu") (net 9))
 (segment (start 93.125 25.875) (end 92.875 25.875) (width 0.127) (layer "B.Cu") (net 18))
 (segment (start 12.875 69.125) (end 13.125 69.125) (width 0.15) (layer "B.Cu") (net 7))
 (segment (start 16.875 78.125) (end 17.125 78.125) (width 0.15) (layer "B.Cu") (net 9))
 (segment (start 17.125 70.125) (end 17.375 70.375) (width 0.15) (layer "B.Cu") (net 7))
 (segment (start 15.125 78.625) (end 15.375 78.375) (width 0.15) (layer "B.Cu") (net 9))
 (segment (start 94.875 25.875) (end 94.625 25.875) (width 0.127) (layer "B.Cu") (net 18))
 (segment (start 15.875 69.125) (end 16.125 69.125) (width 0.15) (layer "B.Cu") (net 7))
 (segment (start 10.875 83.375) (end 10.875 83.125) (width 0.15) (layer "B.Cu") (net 9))
 (segment (start 97.625 25.875) (end 97.375 25.875) (width 0.127) (layer "B.Cu") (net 18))
 (segment (start 15.625 78.375) (end 15.875 78.375) (width 0.15) (layer "B.Cu") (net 9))
 (segment (start 17.875 78.125) (end 18.125 78.125) (width 0.15) (layer "B.Cu") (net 9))
 (segment (start 10.375 84.375) (end 10.625 84.125) (width 0.15) (layer "B.Cu") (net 9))
 (segment (start 12.875 80.375) (end 13.125 80.125) (width 0.15) (layer "B.Cu") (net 9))
 (segment (start 18.125 78.125) (end 18.375 78.125) (width 0.15) (layer "B.Cu") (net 9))
 (segment (start 97.625 26.125) (end 97.625 26.375) (width 0.127) (layer "B.Cu") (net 18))
 (segment (start 14.375 69.125) (end 14.625 69.125) (width 0.15) (layer "B.Cu") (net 7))
 (segment (start 92.625 24.375) (end 92.625 24.125) (width 0.127) (layer "B.Cu") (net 18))
 (segment (start 10.875 82.625) (end 11.125 82.375) (width 0.15) (layer "B.Cu") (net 9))
 (segment (start 10.875 83.875) (end 10.875 83.625) (width 0.15) (layer "B.Cu") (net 9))
 (segment (start 18.125 71.125) (end 18.375 71.375) (width 0.15) (layer "B.Cu") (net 7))
 (segment (start 9.875 65.375) (end 9.875 65.625) (width 0.15) (layer "F.Cu") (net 7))
 (segment (start 92.875 25.875) (end 92.5 25.75) (width 0.127) (layer "B.Cu") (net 18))
 (segment (start 18.625 71.375) (end 18.875 71.375) (width 0.15) (layer "B.Cu") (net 7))
 (segment (start 96.875 25.875) (end 96.625 25.875) (width 0.127) (layer "B.Cu") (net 18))
 (segment (start 15.625 69.125) (end 15.875 69.125) (width 0.15) (layer "B.Cu") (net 7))
 (via (at 9.875 84.875) (size 0.6) (drill 0.3) (layers "F.Cu" "B.Cu") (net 9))
 (via (at 11.125 67.625) (size 0.6) (drill 0.3) (layers "F.Cu" "B.Cu") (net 7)))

